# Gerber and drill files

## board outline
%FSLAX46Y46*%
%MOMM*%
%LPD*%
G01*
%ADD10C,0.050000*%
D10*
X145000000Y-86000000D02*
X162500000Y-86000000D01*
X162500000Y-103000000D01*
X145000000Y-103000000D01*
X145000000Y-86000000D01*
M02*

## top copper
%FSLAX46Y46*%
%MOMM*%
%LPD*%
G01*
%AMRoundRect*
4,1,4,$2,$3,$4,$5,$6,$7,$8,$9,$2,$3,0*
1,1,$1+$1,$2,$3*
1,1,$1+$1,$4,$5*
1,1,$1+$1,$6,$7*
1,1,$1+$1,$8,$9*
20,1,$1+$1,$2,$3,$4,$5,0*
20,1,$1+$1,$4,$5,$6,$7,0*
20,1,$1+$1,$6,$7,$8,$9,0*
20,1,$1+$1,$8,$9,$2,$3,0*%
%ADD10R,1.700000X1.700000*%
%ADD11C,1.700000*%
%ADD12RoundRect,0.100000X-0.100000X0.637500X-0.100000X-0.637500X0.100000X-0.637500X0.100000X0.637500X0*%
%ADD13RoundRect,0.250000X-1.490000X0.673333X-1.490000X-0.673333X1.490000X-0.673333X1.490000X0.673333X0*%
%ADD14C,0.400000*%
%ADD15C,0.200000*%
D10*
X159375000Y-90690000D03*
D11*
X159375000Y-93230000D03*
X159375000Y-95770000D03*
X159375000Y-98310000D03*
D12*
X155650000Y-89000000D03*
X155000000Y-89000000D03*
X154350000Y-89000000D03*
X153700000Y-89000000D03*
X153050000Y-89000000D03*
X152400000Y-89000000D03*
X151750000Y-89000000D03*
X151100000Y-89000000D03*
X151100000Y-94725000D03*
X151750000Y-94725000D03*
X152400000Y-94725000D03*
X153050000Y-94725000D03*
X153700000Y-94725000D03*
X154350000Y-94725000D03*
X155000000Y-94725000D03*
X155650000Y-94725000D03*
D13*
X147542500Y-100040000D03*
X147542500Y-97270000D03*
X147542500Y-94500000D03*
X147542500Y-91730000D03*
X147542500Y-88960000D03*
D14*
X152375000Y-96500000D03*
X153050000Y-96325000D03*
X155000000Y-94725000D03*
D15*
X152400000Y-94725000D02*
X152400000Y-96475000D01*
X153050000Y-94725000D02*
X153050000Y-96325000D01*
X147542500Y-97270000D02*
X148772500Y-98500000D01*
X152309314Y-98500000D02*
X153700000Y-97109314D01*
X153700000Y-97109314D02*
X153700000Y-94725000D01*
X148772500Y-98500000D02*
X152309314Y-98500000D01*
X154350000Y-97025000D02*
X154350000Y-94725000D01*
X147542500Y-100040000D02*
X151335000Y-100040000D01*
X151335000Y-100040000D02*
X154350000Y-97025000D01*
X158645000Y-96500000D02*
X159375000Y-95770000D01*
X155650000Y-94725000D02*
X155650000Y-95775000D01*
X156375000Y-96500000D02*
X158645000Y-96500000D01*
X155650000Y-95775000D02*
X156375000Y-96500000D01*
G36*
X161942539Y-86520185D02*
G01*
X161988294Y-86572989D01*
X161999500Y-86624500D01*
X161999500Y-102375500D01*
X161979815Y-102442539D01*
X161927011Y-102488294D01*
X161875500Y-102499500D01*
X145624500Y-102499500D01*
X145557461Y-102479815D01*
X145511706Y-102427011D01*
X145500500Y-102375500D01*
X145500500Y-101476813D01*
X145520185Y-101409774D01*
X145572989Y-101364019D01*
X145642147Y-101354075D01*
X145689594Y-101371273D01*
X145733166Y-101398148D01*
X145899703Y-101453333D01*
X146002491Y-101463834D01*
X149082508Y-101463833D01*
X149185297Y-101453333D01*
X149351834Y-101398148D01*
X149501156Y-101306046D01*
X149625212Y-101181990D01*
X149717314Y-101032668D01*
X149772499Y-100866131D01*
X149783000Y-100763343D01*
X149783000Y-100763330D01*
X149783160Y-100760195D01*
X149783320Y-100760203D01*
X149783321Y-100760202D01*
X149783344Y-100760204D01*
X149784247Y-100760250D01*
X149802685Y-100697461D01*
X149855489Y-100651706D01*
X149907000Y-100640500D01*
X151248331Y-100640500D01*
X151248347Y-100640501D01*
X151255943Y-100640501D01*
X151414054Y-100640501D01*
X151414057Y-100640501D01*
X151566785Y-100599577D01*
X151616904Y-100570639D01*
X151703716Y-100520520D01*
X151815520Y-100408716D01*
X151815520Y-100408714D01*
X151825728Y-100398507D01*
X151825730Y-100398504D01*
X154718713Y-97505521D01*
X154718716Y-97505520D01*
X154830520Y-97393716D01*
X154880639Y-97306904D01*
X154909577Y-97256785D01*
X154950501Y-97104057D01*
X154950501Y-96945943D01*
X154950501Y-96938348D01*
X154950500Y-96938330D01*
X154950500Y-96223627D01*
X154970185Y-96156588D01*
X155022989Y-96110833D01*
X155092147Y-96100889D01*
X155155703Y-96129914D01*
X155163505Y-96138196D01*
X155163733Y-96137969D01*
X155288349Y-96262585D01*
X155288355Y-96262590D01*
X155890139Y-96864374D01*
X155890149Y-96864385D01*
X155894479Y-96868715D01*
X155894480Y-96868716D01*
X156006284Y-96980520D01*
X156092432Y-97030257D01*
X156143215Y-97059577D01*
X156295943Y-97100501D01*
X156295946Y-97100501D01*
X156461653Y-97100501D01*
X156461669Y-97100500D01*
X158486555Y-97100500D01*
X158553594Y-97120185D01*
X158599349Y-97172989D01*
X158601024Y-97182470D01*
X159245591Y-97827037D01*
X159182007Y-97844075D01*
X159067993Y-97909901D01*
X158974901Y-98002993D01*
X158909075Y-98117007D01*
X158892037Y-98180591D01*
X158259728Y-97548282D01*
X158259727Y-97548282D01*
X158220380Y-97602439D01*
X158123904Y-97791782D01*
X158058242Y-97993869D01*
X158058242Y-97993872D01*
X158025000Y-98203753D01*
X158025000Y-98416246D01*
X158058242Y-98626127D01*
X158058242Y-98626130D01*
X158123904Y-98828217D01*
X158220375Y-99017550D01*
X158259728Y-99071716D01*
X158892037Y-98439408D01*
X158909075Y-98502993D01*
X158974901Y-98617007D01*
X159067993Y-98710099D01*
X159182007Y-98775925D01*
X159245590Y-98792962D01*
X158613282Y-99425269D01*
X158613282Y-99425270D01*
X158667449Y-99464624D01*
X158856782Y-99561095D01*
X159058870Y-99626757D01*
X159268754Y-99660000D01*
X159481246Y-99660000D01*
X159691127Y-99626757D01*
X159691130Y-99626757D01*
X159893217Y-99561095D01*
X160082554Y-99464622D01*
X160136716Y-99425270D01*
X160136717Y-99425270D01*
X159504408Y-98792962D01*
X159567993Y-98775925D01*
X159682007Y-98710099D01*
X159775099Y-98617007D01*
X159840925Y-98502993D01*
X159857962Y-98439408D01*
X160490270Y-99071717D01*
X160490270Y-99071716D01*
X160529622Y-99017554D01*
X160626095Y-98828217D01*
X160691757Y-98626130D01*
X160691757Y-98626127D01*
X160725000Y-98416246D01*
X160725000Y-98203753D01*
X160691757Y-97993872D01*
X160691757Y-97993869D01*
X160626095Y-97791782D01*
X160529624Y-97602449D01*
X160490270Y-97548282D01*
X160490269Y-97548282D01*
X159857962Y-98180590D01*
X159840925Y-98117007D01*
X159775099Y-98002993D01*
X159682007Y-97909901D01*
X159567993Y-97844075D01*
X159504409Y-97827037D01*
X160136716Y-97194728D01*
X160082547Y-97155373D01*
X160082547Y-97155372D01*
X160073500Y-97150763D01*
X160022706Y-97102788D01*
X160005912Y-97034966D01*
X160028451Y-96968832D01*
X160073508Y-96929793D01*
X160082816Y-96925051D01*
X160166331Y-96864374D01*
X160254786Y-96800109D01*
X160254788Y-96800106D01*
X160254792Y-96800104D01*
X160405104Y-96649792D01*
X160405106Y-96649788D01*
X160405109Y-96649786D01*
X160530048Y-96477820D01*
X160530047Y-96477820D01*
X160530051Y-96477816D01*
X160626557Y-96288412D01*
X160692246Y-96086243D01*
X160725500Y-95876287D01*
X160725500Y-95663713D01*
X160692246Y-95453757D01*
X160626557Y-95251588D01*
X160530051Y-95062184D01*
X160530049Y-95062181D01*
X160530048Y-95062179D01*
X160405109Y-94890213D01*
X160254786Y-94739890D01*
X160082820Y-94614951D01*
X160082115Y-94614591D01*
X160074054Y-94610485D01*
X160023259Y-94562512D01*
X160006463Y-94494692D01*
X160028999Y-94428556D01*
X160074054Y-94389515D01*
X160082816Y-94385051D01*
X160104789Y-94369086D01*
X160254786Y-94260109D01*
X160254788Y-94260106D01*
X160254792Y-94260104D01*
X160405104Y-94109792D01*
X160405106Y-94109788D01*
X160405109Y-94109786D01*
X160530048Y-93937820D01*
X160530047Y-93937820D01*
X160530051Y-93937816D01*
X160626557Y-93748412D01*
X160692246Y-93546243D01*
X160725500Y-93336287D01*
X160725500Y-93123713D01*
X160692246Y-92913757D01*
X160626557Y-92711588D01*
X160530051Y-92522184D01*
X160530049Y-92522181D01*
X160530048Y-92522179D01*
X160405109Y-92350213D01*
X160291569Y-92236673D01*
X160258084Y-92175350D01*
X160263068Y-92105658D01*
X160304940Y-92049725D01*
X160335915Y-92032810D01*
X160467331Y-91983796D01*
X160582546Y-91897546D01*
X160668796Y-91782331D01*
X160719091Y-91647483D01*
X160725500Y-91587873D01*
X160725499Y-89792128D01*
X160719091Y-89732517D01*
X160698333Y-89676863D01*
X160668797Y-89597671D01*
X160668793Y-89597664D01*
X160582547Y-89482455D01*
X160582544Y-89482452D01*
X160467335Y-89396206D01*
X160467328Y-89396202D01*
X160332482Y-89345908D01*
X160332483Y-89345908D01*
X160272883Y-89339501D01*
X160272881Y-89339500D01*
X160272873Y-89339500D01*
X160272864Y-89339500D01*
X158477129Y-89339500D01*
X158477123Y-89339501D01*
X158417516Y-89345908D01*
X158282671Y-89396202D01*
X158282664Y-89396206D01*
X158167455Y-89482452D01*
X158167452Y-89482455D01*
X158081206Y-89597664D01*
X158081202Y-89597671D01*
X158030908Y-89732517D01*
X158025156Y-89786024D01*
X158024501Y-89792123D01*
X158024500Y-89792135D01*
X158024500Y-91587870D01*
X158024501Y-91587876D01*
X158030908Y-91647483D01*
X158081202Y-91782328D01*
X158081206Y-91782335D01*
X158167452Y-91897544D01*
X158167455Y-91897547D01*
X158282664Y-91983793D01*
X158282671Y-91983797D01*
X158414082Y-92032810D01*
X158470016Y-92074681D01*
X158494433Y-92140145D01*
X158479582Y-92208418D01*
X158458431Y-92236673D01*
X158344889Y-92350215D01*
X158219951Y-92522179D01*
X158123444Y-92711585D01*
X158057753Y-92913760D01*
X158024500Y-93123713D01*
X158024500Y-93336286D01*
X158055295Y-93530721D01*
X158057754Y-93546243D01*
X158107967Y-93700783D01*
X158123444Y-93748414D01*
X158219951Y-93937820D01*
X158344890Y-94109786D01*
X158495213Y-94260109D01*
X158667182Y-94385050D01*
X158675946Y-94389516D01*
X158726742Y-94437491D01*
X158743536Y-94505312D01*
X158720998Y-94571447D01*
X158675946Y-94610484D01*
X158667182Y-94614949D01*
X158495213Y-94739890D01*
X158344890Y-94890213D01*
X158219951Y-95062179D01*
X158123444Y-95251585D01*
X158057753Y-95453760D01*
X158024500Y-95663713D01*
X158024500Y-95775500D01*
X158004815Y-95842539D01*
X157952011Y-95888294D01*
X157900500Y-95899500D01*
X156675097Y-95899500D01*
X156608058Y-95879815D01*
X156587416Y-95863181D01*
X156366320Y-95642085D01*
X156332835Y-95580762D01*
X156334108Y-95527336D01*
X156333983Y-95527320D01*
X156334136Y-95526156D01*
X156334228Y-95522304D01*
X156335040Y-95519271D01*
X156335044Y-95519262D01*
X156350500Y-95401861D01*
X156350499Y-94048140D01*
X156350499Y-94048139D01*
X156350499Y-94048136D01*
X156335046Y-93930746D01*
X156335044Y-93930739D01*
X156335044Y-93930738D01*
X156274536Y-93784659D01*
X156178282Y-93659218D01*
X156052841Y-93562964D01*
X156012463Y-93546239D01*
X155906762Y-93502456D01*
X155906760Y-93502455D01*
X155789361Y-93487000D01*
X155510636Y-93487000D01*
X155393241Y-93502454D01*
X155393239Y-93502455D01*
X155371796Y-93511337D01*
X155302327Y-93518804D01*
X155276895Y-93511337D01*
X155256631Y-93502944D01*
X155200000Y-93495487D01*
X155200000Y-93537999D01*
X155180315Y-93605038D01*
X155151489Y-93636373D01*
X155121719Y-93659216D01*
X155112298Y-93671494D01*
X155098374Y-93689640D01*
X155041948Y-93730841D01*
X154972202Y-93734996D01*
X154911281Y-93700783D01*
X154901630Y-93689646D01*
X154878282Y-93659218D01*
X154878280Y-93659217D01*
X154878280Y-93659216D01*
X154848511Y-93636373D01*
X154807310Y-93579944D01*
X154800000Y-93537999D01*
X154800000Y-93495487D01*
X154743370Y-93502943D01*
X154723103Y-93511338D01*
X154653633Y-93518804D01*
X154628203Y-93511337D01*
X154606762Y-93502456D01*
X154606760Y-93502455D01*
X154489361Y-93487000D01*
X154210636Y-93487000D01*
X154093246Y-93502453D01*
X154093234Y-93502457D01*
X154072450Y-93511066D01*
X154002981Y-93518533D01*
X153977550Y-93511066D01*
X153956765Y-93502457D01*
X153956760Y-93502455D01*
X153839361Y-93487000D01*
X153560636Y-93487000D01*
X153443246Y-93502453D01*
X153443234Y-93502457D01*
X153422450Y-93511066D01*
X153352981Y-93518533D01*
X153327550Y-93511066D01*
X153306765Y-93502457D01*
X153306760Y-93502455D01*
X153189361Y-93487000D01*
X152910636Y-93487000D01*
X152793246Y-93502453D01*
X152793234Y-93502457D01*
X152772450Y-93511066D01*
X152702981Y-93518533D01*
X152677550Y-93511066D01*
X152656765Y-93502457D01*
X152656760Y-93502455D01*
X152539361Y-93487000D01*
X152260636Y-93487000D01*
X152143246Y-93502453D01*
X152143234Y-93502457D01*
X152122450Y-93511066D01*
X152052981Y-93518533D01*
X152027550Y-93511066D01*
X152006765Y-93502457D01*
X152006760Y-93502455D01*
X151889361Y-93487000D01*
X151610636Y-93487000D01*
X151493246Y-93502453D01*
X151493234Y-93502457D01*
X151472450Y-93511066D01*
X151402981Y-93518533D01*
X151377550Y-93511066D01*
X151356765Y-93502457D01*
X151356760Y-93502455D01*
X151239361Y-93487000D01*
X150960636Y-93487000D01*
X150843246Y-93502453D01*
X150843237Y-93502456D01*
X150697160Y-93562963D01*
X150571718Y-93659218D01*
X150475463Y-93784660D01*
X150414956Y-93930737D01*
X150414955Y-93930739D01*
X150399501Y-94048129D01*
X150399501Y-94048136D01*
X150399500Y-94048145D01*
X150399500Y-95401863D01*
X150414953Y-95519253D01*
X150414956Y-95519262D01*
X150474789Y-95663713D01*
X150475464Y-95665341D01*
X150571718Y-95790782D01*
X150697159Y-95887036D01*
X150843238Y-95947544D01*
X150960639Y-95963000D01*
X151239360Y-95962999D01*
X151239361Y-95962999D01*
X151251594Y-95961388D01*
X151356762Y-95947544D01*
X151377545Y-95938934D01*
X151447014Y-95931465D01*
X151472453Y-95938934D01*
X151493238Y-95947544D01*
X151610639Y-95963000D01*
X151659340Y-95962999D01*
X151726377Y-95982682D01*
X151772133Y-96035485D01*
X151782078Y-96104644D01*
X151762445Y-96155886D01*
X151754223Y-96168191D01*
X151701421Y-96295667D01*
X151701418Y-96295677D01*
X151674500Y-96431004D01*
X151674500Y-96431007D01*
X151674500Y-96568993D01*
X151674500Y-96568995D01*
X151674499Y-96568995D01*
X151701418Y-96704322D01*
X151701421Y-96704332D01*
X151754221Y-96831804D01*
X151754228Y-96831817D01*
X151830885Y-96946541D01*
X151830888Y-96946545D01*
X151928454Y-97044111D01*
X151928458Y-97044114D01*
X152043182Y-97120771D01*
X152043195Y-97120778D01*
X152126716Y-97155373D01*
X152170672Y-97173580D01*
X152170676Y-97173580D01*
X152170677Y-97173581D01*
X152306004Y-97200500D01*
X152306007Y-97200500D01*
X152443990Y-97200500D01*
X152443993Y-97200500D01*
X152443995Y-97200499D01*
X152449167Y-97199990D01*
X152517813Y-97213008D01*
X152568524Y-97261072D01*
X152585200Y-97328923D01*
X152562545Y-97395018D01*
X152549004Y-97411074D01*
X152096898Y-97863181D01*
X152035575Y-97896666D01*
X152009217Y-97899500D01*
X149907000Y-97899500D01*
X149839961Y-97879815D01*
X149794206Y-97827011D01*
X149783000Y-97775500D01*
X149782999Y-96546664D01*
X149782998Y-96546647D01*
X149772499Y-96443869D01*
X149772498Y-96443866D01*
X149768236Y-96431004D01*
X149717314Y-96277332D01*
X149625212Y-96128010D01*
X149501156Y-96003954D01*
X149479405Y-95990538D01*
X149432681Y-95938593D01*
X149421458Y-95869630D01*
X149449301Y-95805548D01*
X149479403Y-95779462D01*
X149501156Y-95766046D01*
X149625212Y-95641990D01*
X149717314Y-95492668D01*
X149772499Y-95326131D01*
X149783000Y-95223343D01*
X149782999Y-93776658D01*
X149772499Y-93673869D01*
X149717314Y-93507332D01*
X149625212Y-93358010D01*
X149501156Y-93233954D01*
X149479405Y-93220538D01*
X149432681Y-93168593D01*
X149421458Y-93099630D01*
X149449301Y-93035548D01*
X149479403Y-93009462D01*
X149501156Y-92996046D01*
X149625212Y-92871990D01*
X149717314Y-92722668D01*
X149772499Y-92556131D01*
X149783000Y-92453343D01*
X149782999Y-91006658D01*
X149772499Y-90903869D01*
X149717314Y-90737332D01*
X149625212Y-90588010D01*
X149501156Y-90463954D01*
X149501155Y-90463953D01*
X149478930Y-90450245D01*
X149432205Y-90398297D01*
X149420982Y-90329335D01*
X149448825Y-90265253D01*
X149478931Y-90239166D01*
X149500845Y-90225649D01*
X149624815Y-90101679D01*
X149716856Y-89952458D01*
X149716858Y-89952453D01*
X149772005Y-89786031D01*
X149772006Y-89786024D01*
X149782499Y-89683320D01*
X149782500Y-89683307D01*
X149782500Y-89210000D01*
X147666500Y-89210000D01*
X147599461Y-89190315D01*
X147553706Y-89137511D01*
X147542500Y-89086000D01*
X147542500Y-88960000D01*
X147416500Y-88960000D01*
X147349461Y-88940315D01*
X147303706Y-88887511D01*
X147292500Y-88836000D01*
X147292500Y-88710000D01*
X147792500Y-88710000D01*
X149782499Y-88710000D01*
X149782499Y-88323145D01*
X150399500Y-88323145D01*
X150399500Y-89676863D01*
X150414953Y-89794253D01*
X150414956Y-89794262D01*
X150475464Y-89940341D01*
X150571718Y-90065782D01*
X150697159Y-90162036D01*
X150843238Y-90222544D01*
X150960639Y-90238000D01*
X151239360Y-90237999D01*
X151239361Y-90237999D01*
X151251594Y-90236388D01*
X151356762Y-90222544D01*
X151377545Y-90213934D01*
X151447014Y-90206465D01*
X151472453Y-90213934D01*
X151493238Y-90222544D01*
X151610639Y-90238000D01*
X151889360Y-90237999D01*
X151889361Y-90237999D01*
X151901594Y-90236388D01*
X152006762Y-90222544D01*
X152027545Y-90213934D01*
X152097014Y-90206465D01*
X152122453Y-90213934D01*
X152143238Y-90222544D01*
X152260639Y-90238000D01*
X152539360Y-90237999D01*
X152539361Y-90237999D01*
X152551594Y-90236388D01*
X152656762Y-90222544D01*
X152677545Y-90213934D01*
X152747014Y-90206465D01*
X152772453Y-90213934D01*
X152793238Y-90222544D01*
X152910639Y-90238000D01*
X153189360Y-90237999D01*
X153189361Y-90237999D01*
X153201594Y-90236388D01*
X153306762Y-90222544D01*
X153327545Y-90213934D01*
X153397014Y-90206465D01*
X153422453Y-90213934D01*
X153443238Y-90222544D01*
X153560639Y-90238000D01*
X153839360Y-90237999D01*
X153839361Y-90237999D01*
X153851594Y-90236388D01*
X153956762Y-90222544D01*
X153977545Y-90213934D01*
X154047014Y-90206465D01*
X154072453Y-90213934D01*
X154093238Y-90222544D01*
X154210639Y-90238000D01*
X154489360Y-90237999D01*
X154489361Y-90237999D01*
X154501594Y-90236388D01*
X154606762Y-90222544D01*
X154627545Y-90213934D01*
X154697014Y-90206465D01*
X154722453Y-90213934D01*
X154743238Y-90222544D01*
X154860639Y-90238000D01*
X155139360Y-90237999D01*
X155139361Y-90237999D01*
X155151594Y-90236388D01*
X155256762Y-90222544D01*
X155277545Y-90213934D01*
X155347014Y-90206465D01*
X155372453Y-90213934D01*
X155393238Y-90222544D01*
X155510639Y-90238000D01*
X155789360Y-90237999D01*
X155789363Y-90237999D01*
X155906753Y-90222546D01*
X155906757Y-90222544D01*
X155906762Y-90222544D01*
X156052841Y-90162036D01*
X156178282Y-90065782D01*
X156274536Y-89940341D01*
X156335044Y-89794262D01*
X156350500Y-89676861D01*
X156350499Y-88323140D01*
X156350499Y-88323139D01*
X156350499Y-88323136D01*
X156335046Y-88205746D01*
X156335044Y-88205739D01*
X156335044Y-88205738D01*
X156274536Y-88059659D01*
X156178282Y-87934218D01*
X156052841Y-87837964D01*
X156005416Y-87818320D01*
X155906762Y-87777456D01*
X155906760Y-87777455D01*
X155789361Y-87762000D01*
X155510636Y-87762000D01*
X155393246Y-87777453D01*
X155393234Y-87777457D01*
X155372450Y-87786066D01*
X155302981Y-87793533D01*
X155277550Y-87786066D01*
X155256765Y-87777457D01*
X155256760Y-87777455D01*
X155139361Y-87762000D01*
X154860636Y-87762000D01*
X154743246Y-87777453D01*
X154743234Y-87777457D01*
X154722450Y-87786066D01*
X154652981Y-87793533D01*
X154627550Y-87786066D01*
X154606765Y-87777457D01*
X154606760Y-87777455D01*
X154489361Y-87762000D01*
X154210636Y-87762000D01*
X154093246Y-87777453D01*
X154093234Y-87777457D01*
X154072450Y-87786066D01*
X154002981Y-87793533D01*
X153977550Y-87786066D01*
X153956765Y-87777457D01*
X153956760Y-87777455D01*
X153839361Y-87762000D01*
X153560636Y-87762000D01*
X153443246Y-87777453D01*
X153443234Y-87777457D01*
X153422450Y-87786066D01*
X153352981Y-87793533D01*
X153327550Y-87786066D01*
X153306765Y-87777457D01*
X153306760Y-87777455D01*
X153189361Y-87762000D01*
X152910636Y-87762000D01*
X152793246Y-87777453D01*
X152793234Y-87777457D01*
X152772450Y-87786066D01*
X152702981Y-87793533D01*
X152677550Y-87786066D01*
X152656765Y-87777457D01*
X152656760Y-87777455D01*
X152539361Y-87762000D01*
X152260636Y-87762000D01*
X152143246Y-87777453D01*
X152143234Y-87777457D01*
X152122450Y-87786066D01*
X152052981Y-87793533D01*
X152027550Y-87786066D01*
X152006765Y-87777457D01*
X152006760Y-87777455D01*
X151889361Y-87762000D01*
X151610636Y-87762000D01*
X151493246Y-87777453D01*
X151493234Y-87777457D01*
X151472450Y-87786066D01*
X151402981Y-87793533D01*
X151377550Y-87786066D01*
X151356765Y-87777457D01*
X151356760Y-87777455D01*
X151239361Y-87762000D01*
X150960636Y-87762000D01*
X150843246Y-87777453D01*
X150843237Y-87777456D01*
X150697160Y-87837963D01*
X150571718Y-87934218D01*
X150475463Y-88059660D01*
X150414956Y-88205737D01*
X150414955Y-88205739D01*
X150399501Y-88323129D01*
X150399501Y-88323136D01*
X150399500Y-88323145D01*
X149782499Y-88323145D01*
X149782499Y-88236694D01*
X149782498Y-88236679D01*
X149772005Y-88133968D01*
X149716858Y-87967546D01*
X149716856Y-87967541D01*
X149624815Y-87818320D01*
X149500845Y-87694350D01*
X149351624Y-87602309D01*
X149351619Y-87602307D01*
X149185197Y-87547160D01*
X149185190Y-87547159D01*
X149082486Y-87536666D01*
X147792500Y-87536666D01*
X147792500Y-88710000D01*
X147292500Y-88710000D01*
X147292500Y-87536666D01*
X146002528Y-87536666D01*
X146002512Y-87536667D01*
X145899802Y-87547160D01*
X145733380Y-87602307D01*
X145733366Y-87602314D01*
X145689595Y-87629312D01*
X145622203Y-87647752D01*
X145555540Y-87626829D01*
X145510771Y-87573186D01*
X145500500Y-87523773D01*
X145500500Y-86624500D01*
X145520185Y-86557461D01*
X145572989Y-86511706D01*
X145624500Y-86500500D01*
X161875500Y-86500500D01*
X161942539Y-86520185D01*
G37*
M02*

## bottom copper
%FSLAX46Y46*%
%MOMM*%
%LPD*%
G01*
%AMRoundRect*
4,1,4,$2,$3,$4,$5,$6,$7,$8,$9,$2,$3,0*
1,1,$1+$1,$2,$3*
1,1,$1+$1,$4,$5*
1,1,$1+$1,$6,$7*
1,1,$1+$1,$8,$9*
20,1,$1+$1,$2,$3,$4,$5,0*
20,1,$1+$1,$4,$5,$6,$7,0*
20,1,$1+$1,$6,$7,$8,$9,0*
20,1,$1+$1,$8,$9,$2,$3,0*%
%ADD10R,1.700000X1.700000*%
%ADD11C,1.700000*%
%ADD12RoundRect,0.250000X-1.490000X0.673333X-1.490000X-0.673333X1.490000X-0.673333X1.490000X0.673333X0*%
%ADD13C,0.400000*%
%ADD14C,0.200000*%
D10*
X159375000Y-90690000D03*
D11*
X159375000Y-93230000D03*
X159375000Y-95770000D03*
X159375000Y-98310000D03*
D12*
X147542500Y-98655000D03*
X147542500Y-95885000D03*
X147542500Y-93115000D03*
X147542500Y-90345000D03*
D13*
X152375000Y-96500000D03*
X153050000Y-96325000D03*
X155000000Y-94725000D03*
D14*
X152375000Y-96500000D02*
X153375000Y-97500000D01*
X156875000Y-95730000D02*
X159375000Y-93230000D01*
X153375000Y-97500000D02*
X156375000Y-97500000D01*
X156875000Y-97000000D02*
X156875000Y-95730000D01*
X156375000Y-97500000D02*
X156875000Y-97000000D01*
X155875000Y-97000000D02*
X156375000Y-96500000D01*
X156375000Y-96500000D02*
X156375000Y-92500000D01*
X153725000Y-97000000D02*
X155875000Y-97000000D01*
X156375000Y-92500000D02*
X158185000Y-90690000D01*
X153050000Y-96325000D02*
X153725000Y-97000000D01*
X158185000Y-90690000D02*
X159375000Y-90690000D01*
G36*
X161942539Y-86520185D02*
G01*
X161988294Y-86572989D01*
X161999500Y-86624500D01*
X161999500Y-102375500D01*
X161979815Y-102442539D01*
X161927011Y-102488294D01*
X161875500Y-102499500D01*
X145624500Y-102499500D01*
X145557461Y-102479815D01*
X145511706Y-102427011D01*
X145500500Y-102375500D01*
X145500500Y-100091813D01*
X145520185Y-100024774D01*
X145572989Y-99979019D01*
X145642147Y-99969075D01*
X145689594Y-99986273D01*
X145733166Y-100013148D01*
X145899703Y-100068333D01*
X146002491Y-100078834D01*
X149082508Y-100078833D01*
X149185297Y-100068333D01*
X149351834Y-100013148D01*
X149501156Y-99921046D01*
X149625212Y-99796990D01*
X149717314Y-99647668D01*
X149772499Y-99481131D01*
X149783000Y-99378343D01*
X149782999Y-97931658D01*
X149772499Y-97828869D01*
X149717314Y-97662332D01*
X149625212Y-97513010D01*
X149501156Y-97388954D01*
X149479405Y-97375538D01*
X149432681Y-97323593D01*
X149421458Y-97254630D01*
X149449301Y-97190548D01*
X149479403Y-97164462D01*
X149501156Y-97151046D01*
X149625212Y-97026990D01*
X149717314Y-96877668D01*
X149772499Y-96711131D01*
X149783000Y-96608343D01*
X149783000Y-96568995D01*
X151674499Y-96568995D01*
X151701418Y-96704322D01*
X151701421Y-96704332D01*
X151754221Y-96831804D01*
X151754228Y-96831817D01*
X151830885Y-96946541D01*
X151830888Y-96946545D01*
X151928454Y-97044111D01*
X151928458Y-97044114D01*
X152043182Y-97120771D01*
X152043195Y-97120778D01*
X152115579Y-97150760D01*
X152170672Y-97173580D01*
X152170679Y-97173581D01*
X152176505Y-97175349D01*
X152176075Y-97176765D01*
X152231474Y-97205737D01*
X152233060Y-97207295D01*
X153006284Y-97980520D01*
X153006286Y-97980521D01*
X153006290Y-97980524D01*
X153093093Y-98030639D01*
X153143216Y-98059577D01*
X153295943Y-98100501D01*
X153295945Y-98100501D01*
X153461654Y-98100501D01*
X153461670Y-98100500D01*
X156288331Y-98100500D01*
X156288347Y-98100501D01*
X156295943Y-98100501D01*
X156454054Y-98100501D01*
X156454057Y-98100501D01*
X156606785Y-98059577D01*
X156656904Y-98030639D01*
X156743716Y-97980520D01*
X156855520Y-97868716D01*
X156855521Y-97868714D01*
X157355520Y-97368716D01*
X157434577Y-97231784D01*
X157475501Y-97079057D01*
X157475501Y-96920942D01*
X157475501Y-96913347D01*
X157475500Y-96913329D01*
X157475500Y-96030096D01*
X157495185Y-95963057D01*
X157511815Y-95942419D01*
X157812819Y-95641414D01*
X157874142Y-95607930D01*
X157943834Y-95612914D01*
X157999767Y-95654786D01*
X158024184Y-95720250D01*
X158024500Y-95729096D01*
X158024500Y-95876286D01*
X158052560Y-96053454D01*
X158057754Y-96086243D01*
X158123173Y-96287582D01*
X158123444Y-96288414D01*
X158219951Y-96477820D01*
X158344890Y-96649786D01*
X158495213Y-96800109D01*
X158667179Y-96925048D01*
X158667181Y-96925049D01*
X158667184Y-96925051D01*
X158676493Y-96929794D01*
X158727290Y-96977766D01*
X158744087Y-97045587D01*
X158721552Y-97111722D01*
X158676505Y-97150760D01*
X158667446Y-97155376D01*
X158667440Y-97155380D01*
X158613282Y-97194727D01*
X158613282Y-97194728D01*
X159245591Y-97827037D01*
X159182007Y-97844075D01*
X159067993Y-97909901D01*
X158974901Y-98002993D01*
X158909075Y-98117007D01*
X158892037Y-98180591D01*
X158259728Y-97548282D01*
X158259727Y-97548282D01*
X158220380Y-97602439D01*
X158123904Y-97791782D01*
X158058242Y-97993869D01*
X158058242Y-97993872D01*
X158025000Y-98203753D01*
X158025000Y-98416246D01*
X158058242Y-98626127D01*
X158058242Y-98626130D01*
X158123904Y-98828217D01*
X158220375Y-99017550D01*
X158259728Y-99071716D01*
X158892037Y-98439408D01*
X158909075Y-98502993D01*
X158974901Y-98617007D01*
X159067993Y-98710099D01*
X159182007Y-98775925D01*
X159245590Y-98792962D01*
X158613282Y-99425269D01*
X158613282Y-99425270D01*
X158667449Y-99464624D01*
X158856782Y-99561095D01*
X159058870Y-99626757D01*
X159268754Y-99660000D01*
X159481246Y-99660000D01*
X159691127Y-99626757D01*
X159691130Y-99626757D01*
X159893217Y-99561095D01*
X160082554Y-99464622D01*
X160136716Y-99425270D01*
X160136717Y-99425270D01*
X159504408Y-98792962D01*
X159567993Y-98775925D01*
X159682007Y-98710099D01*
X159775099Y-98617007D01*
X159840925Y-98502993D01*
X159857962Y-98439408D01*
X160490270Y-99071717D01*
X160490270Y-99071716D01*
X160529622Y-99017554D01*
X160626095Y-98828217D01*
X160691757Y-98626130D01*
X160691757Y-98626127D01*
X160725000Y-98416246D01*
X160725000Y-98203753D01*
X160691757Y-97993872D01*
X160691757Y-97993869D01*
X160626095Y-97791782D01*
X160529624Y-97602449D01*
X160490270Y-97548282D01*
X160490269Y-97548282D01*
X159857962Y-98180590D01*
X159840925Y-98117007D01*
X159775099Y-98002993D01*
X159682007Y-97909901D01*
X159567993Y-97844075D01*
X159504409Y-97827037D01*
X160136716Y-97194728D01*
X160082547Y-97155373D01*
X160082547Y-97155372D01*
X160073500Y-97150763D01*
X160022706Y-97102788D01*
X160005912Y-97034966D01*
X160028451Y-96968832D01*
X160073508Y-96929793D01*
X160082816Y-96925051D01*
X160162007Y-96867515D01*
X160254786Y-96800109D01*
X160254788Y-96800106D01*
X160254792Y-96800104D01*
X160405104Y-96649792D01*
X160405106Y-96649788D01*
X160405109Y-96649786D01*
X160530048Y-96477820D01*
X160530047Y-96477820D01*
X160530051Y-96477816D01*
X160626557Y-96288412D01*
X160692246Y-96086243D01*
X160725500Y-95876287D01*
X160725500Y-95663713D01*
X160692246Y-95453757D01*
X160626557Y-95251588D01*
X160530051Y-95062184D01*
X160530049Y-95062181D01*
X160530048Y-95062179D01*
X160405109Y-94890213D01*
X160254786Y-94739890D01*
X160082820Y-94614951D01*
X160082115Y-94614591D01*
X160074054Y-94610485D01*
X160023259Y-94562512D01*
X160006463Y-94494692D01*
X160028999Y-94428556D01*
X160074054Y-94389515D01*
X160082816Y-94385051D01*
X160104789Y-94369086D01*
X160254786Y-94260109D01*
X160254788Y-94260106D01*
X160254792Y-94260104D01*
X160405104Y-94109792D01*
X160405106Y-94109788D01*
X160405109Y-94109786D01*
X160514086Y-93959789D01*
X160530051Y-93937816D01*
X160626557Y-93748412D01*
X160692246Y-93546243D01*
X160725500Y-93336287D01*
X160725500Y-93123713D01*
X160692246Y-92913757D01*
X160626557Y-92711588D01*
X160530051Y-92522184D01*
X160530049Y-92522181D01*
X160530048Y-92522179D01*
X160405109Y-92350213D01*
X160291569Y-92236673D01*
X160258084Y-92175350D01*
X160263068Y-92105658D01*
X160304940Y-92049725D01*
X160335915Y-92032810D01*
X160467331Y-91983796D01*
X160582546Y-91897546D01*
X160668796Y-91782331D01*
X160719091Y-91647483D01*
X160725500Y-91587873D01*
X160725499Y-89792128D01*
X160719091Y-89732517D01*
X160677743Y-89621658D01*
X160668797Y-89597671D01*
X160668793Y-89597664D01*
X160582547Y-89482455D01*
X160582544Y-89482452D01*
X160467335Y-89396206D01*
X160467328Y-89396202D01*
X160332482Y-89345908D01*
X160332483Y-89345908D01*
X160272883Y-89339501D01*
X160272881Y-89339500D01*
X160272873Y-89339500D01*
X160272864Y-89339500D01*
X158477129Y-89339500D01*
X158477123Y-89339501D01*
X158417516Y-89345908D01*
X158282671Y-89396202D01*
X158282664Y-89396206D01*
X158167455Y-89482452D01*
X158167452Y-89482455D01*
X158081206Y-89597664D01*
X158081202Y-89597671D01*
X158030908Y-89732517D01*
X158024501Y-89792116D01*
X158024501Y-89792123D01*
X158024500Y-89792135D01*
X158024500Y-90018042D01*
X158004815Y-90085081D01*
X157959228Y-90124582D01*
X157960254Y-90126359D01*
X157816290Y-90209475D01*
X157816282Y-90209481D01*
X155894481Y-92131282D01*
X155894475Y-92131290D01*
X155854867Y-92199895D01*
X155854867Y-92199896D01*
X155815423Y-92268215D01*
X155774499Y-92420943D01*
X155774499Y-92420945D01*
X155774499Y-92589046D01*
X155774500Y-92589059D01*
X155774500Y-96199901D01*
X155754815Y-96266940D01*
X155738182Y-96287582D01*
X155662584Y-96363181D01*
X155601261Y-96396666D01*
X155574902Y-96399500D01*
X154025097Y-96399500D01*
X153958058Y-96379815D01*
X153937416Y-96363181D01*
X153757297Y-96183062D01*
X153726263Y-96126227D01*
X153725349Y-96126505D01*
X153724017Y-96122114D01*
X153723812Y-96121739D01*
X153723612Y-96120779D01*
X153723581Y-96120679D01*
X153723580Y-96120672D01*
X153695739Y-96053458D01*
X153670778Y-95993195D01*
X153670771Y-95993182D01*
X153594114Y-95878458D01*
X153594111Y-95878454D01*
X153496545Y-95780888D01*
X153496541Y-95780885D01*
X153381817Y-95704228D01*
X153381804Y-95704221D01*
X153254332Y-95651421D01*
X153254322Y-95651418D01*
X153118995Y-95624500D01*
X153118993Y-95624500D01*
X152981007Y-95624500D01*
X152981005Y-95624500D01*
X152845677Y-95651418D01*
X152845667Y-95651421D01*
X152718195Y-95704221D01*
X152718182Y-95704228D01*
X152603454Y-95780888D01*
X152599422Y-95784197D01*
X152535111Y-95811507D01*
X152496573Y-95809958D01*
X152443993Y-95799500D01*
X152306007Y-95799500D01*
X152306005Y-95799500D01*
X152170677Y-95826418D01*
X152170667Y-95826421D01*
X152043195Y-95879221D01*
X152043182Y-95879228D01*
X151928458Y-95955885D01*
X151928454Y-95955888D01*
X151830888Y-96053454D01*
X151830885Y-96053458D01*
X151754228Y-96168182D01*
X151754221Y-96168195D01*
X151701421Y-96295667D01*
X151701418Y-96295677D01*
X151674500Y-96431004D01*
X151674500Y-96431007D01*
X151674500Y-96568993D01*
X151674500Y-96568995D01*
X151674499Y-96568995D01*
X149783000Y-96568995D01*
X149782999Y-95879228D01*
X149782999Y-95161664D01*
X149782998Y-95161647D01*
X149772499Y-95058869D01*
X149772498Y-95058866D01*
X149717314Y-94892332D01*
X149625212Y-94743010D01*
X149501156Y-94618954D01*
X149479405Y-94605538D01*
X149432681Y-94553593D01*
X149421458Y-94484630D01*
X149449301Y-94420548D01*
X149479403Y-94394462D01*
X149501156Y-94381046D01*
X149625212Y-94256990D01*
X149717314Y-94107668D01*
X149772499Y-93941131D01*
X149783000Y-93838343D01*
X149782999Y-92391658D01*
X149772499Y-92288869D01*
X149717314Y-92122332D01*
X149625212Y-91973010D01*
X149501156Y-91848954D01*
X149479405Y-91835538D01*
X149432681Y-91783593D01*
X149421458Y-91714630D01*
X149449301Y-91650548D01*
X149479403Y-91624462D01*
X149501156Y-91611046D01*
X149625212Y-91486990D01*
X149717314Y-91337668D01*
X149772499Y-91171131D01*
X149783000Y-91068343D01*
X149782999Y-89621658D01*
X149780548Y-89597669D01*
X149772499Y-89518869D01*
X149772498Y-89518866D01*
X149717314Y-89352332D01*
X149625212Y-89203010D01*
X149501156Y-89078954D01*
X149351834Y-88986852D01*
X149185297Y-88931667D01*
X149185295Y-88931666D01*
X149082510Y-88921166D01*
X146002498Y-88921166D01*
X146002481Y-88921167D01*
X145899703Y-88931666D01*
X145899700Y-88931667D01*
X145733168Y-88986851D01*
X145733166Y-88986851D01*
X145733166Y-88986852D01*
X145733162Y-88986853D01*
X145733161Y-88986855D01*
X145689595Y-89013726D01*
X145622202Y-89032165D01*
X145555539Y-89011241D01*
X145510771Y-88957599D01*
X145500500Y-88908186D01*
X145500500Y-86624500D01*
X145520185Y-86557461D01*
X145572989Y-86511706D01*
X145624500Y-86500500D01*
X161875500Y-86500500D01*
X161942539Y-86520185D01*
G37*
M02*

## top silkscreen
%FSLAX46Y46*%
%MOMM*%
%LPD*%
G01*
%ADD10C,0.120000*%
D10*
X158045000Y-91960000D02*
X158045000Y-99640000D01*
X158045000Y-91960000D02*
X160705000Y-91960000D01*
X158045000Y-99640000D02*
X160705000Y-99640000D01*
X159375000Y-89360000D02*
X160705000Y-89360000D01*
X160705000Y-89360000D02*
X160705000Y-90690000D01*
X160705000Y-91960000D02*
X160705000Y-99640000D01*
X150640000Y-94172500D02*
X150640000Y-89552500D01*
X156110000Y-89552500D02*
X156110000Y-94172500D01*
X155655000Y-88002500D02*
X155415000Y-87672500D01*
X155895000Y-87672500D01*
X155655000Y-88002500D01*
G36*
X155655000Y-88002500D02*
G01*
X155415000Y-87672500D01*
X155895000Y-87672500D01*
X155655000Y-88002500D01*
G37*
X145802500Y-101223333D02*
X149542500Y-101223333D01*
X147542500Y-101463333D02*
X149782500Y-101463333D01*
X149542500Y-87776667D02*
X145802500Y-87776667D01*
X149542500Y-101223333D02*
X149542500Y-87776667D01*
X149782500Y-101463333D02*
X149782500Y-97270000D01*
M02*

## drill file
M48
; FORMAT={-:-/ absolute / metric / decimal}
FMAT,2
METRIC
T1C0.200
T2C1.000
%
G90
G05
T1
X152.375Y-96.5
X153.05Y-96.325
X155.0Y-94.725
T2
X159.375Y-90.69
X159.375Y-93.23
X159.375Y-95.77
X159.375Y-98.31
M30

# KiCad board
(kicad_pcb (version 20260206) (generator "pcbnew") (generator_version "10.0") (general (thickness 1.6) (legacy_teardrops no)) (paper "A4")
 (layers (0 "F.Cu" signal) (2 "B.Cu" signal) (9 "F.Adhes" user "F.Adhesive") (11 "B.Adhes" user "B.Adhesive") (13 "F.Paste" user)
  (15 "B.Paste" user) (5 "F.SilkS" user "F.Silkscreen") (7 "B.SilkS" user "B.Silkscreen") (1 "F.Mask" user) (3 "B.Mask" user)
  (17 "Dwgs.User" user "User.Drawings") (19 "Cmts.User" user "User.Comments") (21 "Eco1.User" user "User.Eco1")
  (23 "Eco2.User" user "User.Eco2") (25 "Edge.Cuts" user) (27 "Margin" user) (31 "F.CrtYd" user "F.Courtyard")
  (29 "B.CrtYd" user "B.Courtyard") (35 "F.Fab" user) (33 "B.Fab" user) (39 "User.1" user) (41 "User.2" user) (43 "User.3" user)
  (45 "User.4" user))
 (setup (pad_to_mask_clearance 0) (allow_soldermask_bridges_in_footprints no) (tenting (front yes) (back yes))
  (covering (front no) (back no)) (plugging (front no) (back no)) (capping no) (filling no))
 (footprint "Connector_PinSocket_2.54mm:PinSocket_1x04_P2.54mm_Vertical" (layer "F.Cu") (at 159.375 90.69)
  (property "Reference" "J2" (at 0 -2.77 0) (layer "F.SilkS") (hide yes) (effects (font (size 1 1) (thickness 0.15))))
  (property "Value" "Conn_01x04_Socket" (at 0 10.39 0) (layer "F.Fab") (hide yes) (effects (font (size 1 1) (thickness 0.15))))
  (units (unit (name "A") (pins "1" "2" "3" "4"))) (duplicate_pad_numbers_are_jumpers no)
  (fp_line (start -1.33 1.27) (end -1.33 8.95) (stroke (width 0.12) (type solid)) (layer "F.SilkS"))
  (fp_line (start -1.33 1.27) (end 1.33 1.27) (stroke (width 0.12) (type solid)) (layer "F.SilkS"))
  (fp_line (start -1.33 8.95) (end 1.33 8.95) (stroke (width 0.12) (type solid)) (layer "F.SilkS"))
  (fp_line (start 0 -1.33) (end 1.33 -1.33) (stroke (width 0.12) (type solid)) (layer "F.SilkS"))
  (fp_line (start 1.33 -1.33) (end 1.33 0) (stroke (width 0.12) (type solid)) (layer "F.SilkS"))
  (fp_line (start 1.33 1.27) (end 1.33 8.95) (stroke (width 0.12) (type solid)) (layer "F.SilkS"))
  (pad "1" thru_hole rect (at 0 0) (size 1.7 1.7) (drill 1) (layers "*.Cu" "*.Mask") (remove_unused_layers no) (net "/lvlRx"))
  (pad "2" thru_hole circle (at 0 2.54) (size 1.7 1.7) (drill 1) (layers "*.Cu" "*.Mask") (remove_unused_layers no) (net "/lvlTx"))
  (pad "3" thru_hole circle (at 0 5.08) (size 1.7 1.7) (drill 1) (layers "*.Cu" "*.Mask") (remove_unused_layers no) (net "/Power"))
  (pad "4" thru_hole circle (at 0 7.62) (size 1.7 1.7) (drill 1) (layers "*.Cu" "*.Mask") (remove_unused_layers no) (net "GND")))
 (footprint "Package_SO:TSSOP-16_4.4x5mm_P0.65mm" (layer "F.Cu") (at 153.375 91.8625 -90)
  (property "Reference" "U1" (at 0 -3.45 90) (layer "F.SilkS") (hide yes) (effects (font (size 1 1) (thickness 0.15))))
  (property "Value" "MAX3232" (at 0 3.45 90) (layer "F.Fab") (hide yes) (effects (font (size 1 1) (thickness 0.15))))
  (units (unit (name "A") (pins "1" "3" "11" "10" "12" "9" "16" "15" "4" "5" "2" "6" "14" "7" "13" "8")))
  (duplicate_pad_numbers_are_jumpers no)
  (fp_line (start 2.31 2.735) (end -2.31 2.735) (stroke (width 0.12) (type solid)) (layer "F.SilkS"))
  (fp_line (start -2.31 -2.735) (end 2.31 -2.735) (stroke (width 0.12) (type solid)) (layer "F.SilkS"))
  (fp_poly (pts (xy -3.86 -2.28) (xy -4.19 -2.04) (xy -4.19 -2.52)) (stroke (width 0.12) (type solid)) (fill yes) (layer "F.SilkS"))
  (pad "1" smd roundrect (at -2.8625 -2.275 270) (size 1.475 0.4) (layers "F.Cu" "F.Mask" "F.Paste") (roundrect_rratio 0.25)
   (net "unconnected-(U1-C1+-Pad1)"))
  (pad "2" smd roundrect (at -2.8625 -1.625 270) (size 1.475 0.4) (layers "F.Cu" "F.Mask" "F.Paste") (roundrect_rratio 0.25)
   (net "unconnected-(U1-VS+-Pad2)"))
  (pad "3" smd roundrect (at -2.8625 -0.975 270) (size 1.475 0.4) (layers "F.Cu" "F.Mask" "F.Paste") (roundrect_rratio 0.25)
   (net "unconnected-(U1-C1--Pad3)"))
  (pad "4" smd roundrect (at -2.8625 -0.325 270) (size 1.475 0.4) (layers "F.Cu" "F.Mask" "F.Paste") (roundrect_rratio 0.25)
   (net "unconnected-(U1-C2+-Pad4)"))
  (pad "5" smd roundrect (at -2.8625 0.325 270) (size 1.475 0.4) (layers "F.Cu" "F.Mask" "F.Paste") (roundrect_rratio 0.25)
   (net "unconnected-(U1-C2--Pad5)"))
  (pad "6" smd roundrect (at -2.8625 0.975 270) (size 1.475 0.4) (layers "F.Cu" "F.Mask" "F.Paste") (roundrect_rratio 0.25)
   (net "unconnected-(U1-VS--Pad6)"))
  (pad "7" smd roundrect (at -2.8625 1.625 270) (size 1.475 0.4) (layers "F.Cu" "F.Mask" "F.Paste") (roundrect_rratio 0.25)
   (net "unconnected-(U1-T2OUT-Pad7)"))
  (pad "8" smd roundrect (at -2.8625 2.275 270) (size 1.475 0.4) (layers "F.Cu" "F.Mask" "F.Paste") (roundrect_rratio 0.25)
   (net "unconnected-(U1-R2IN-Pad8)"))
  (pad "9" smd roundrect (at 2.8625 2.275 270) (size 1.475 0.4) (layers "F.Cu" "F.Mask" "F.Paste") (roundrect_rratio 0.25)
   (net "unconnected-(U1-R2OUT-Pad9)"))
  (pad "10" smd roundrect (at 2.8625 1.625 270) (size 1.475 0.4) (layers "F.Cu" "F.Mask" "F.Paste") (roundrect_rratio 0.25)
   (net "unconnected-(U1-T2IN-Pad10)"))
  (pad "11" smd roundrect (at 2.8625 0.975 270) (size 1.475 0.4) (layers "F.Cu" "F.Mask" "F.Paste") (roundrect_rratio 0.25) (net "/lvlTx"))
  (pad "12" smd roundrect (at 2.8625 0.325 270) (size 1.475 0.4) (layers "F.Cu" "F.Mask" "F.Paste") (roundrect_rratio 0.25) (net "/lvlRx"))
  (pad "13" smd roundrect (at 2.8625 -0.325 270) (size 1.475 0.4) (layers "F.Cu" "F.Mask" "F.Paste") (roundrect_rratio 0.25)
   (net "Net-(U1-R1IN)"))
  (pad "14" smd roundrect (at 2.8625 -0.975 270) (size 1.475 0.4) (layers "F.Cu" "F.Mask" "F.Paste") (roundrect_rratio 0.25)
   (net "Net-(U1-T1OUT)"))
  (pad "15" smd roundrect (at 2.8625 -1.625 270) (size 1.475 0.4) (layers "F.Cu" "F.Mask" "F.Paste") (roundrect_rratio 0.25) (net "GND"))
  (pad "16" smd roundrect (at 2.8625 -2.275 270) (size 1.475 0.4) (layers "F.Cu" "F.Mask" "F.Paste") (roundrect_rratio 0.25) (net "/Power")))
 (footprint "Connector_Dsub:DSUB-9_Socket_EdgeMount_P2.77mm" (layer "F.Cu") (at 147.5425 94.5 -90)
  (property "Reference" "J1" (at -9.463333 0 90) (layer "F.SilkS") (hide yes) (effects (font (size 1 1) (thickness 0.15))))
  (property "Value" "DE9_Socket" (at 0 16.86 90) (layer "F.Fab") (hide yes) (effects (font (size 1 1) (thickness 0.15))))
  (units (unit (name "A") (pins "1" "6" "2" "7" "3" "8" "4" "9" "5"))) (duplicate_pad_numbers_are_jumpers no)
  (fp_line (start 6.723333 1.74) (end 6.723333 -2) (stroke (width 0.12) (type solid)) (layer "F.SilkS"))
  (fp_line (start 6.963333 0) (end 6.963333 -2.24) (stroke (width 0.12) (type solid)) (layer "F.SilkS"))
  (fp_line (start -6.723333 -2) (end -6.723333 1.74) (stroke (width 0.12) (type solid)) (layer "F.SilkS"))
  (fp_line (start 6.723333 -2) (end -6.723333 -2) (stroke (width 0.12) (type solid)) (layer "F.SilkS"))
  (fp_line (start 6.963333 -2.24) (end 2.77 -2.24) (stroke (width 0.12) (type solid)) (layer "F.SilkS"))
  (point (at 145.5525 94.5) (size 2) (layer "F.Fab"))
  (pad "1" smd roundrect (at 5.54 0 270) (size 1.846667 3.48) (layers "F.Cu" "F.Mask" "F.Paste") (roundrect_rratio 0.135379)
   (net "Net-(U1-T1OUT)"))
  (pad "2" smd roundrect (at 2.77 0 270) (size 1.846667 3.48) (layers "F.Cu" "F.Mask" "F.Paste") (roundrect_rratio 0.135379)
   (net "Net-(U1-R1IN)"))
  (pad "3" smd roundrect (at 0 0 270) (size 1.846667 3.48) (layers "F.Cu" "F.Mask" "F.Paste") (roundrect_rratio 0.135379)
   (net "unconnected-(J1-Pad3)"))
  (pad "4" smd roundrect (at -2.77 0 270) (size 1.846667 3.48) (layers "F.Cu" "F.Mask" "F.Paste") (roundrect_rratio 0.135379)
   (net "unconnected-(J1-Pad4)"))
  (pad "5" smd roundrect (at -5.54 0 270) (size 1.846667 3.48) (layers "F.Cu" "F.Mask" "F.Paste") (roundrect_rratio 0.135379) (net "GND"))
  (pad "6" smd roundrect (at 4.155 0 270) (size 1.846667 3.48) (layers "B.Cu" "B.Mask" "B.Paste") (roundrect_rratio 0.135379)
   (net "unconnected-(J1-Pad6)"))
  (pad "7" smd roundrect (at 1.385 0 270) (size 1.846667 3.48) (layers "B.Cu" "B.Mask" "B.Paste") (roundrect_rratio 0.135379)
   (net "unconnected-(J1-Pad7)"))
  (pad "8" smd roundrect (at -1.385 0 270) (size 1.846667 3.48) (layers "B.Cu" "B.Mask" "B.Paste") (roundrect_rratio 0.135379)
   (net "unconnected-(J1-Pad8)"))
  (pad "9" smd roundrect (at -4.155 0 270) (size 1.846667 3.48) (layers "B.Cu" "B.Mask" "B.Paste") (roundrect_rratio 0.135379)
   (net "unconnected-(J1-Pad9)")))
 (gr_rect (start 145 86) (end 162.5 103) (stroke (width 0.05) (type default)) (fill no) (layer "Edge.Cuts"))
 (segment (start 152.4 94.725) (end 152.4 96.475) (width 0.2) (layer "F.Cu") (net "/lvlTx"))
 (via (at 152.375 96.5) (size 0.4) (drill 0.2) (layers "F.Cu" "B.Cu") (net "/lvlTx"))
 (segment (start 152.375 96.5) (end 153.375 97.5) (width 0.2) (layer "B.Cu") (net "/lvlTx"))
 (segment (start 156.875 95.73) (end 159.375 93.23) (width 0.2) (layer "B.Cu") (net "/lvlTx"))
 (segment (start 153.375 97.5) (end 156.375 97.5) (width 0.2) (layer "B.Cu") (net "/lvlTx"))
 (segment (start 156.875 97) (end 156.875 95.73) (width 0.2) (layer "B.Cu") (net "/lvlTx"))
 (segment (start 156.375 97.5) (end 156.875 97) (width 0.2) (layer "B.Cu") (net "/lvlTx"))
 (segment (start 153.05 94.725) (end 153.05 96.325) (width 0.2) (layer "F.Cu") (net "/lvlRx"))
 (via (at 153.05 96.325) (size 0.4) (drill 0.2) (layers "F.Cu" "B.Cu") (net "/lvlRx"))
 (segment (start 155.875 97) (end 156.375 96.5) (width 0.2) (layer "B.Cu") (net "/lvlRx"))
 (segment (start 156.375 96.5) (end 156.375 92.5) (width 0.2) (layer "B.Cu") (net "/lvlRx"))
 (segment (start 153.725 97) (end 155.875 97) (width 0.2) (layer "B.Cu") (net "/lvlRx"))
 (segment (start 156.375 92.5) (end 158.185 90.69) (width 0.2) (layer "B.Cu") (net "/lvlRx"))
 (segment (start 153.05 96.325) (end 153.725 97) (width 0.2) (layer "B.Cu") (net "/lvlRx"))
 (segment (start 158.185 90.69) (end 159.375 90.69) (width 0.2) (layer "B.Cu") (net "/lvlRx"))
 (segment (start 147.5425 97.27) (end 148.7725 98.5) (width 0.2) (layer "F.Cu") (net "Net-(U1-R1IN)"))
 (segment (start 152.309314 98.5) (end 153.7 97.109314) (width 0.2) (layer "F.Cu") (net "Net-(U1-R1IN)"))
 (segment (start 153.7 97.109314) (end 153.7 94.725) (width 0.2) (layer "F.Cu") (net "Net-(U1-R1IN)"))
 (segment (start 148.7725 98.5) (end 152.309314 98.5) (width 0.2) (layer "F.Cu") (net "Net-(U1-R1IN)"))
 (segment (start 154.35 97.025) (end 154.35 94.725) (width 0.2) (layer "F.Cu") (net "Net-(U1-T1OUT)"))
 (segment (start 147.5425 100.04) (end 151.335 100.04) (width 0.2) (layer "F.Cu") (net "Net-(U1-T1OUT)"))
 (segment (start 151.335 100.04) (end 154.35 97.025) (width 0.2) (layer "F.Cu") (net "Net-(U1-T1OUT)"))
 (via (at 155 94.725) (size 0.4) (drill 0.2) (layers "F.Cu" "B.Cu") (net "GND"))
 (segment (start 158.645 96.5) (end 159.375 95.77) (width 0.2) (layer "F.Cu") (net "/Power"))
 (segment (start 155.65 94.725) (end 155.65 95.775) (width 0.2) (layer "F.Cu") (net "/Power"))
 (segment (start 156.375 96.5) (end 158.645 96.5) (width 0.2) (layer "F.Cu") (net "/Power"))
 (segment (start 155.65 95.775) (end 156.375 96.5) (width 0.2) (layer "F.Cu") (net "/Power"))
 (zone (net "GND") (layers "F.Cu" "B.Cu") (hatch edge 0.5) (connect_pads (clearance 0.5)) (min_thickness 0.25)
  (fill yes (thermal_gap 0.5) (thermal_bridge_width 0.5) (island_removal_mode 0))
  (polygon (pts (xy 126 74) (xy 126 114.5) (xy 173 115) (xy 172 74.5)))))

